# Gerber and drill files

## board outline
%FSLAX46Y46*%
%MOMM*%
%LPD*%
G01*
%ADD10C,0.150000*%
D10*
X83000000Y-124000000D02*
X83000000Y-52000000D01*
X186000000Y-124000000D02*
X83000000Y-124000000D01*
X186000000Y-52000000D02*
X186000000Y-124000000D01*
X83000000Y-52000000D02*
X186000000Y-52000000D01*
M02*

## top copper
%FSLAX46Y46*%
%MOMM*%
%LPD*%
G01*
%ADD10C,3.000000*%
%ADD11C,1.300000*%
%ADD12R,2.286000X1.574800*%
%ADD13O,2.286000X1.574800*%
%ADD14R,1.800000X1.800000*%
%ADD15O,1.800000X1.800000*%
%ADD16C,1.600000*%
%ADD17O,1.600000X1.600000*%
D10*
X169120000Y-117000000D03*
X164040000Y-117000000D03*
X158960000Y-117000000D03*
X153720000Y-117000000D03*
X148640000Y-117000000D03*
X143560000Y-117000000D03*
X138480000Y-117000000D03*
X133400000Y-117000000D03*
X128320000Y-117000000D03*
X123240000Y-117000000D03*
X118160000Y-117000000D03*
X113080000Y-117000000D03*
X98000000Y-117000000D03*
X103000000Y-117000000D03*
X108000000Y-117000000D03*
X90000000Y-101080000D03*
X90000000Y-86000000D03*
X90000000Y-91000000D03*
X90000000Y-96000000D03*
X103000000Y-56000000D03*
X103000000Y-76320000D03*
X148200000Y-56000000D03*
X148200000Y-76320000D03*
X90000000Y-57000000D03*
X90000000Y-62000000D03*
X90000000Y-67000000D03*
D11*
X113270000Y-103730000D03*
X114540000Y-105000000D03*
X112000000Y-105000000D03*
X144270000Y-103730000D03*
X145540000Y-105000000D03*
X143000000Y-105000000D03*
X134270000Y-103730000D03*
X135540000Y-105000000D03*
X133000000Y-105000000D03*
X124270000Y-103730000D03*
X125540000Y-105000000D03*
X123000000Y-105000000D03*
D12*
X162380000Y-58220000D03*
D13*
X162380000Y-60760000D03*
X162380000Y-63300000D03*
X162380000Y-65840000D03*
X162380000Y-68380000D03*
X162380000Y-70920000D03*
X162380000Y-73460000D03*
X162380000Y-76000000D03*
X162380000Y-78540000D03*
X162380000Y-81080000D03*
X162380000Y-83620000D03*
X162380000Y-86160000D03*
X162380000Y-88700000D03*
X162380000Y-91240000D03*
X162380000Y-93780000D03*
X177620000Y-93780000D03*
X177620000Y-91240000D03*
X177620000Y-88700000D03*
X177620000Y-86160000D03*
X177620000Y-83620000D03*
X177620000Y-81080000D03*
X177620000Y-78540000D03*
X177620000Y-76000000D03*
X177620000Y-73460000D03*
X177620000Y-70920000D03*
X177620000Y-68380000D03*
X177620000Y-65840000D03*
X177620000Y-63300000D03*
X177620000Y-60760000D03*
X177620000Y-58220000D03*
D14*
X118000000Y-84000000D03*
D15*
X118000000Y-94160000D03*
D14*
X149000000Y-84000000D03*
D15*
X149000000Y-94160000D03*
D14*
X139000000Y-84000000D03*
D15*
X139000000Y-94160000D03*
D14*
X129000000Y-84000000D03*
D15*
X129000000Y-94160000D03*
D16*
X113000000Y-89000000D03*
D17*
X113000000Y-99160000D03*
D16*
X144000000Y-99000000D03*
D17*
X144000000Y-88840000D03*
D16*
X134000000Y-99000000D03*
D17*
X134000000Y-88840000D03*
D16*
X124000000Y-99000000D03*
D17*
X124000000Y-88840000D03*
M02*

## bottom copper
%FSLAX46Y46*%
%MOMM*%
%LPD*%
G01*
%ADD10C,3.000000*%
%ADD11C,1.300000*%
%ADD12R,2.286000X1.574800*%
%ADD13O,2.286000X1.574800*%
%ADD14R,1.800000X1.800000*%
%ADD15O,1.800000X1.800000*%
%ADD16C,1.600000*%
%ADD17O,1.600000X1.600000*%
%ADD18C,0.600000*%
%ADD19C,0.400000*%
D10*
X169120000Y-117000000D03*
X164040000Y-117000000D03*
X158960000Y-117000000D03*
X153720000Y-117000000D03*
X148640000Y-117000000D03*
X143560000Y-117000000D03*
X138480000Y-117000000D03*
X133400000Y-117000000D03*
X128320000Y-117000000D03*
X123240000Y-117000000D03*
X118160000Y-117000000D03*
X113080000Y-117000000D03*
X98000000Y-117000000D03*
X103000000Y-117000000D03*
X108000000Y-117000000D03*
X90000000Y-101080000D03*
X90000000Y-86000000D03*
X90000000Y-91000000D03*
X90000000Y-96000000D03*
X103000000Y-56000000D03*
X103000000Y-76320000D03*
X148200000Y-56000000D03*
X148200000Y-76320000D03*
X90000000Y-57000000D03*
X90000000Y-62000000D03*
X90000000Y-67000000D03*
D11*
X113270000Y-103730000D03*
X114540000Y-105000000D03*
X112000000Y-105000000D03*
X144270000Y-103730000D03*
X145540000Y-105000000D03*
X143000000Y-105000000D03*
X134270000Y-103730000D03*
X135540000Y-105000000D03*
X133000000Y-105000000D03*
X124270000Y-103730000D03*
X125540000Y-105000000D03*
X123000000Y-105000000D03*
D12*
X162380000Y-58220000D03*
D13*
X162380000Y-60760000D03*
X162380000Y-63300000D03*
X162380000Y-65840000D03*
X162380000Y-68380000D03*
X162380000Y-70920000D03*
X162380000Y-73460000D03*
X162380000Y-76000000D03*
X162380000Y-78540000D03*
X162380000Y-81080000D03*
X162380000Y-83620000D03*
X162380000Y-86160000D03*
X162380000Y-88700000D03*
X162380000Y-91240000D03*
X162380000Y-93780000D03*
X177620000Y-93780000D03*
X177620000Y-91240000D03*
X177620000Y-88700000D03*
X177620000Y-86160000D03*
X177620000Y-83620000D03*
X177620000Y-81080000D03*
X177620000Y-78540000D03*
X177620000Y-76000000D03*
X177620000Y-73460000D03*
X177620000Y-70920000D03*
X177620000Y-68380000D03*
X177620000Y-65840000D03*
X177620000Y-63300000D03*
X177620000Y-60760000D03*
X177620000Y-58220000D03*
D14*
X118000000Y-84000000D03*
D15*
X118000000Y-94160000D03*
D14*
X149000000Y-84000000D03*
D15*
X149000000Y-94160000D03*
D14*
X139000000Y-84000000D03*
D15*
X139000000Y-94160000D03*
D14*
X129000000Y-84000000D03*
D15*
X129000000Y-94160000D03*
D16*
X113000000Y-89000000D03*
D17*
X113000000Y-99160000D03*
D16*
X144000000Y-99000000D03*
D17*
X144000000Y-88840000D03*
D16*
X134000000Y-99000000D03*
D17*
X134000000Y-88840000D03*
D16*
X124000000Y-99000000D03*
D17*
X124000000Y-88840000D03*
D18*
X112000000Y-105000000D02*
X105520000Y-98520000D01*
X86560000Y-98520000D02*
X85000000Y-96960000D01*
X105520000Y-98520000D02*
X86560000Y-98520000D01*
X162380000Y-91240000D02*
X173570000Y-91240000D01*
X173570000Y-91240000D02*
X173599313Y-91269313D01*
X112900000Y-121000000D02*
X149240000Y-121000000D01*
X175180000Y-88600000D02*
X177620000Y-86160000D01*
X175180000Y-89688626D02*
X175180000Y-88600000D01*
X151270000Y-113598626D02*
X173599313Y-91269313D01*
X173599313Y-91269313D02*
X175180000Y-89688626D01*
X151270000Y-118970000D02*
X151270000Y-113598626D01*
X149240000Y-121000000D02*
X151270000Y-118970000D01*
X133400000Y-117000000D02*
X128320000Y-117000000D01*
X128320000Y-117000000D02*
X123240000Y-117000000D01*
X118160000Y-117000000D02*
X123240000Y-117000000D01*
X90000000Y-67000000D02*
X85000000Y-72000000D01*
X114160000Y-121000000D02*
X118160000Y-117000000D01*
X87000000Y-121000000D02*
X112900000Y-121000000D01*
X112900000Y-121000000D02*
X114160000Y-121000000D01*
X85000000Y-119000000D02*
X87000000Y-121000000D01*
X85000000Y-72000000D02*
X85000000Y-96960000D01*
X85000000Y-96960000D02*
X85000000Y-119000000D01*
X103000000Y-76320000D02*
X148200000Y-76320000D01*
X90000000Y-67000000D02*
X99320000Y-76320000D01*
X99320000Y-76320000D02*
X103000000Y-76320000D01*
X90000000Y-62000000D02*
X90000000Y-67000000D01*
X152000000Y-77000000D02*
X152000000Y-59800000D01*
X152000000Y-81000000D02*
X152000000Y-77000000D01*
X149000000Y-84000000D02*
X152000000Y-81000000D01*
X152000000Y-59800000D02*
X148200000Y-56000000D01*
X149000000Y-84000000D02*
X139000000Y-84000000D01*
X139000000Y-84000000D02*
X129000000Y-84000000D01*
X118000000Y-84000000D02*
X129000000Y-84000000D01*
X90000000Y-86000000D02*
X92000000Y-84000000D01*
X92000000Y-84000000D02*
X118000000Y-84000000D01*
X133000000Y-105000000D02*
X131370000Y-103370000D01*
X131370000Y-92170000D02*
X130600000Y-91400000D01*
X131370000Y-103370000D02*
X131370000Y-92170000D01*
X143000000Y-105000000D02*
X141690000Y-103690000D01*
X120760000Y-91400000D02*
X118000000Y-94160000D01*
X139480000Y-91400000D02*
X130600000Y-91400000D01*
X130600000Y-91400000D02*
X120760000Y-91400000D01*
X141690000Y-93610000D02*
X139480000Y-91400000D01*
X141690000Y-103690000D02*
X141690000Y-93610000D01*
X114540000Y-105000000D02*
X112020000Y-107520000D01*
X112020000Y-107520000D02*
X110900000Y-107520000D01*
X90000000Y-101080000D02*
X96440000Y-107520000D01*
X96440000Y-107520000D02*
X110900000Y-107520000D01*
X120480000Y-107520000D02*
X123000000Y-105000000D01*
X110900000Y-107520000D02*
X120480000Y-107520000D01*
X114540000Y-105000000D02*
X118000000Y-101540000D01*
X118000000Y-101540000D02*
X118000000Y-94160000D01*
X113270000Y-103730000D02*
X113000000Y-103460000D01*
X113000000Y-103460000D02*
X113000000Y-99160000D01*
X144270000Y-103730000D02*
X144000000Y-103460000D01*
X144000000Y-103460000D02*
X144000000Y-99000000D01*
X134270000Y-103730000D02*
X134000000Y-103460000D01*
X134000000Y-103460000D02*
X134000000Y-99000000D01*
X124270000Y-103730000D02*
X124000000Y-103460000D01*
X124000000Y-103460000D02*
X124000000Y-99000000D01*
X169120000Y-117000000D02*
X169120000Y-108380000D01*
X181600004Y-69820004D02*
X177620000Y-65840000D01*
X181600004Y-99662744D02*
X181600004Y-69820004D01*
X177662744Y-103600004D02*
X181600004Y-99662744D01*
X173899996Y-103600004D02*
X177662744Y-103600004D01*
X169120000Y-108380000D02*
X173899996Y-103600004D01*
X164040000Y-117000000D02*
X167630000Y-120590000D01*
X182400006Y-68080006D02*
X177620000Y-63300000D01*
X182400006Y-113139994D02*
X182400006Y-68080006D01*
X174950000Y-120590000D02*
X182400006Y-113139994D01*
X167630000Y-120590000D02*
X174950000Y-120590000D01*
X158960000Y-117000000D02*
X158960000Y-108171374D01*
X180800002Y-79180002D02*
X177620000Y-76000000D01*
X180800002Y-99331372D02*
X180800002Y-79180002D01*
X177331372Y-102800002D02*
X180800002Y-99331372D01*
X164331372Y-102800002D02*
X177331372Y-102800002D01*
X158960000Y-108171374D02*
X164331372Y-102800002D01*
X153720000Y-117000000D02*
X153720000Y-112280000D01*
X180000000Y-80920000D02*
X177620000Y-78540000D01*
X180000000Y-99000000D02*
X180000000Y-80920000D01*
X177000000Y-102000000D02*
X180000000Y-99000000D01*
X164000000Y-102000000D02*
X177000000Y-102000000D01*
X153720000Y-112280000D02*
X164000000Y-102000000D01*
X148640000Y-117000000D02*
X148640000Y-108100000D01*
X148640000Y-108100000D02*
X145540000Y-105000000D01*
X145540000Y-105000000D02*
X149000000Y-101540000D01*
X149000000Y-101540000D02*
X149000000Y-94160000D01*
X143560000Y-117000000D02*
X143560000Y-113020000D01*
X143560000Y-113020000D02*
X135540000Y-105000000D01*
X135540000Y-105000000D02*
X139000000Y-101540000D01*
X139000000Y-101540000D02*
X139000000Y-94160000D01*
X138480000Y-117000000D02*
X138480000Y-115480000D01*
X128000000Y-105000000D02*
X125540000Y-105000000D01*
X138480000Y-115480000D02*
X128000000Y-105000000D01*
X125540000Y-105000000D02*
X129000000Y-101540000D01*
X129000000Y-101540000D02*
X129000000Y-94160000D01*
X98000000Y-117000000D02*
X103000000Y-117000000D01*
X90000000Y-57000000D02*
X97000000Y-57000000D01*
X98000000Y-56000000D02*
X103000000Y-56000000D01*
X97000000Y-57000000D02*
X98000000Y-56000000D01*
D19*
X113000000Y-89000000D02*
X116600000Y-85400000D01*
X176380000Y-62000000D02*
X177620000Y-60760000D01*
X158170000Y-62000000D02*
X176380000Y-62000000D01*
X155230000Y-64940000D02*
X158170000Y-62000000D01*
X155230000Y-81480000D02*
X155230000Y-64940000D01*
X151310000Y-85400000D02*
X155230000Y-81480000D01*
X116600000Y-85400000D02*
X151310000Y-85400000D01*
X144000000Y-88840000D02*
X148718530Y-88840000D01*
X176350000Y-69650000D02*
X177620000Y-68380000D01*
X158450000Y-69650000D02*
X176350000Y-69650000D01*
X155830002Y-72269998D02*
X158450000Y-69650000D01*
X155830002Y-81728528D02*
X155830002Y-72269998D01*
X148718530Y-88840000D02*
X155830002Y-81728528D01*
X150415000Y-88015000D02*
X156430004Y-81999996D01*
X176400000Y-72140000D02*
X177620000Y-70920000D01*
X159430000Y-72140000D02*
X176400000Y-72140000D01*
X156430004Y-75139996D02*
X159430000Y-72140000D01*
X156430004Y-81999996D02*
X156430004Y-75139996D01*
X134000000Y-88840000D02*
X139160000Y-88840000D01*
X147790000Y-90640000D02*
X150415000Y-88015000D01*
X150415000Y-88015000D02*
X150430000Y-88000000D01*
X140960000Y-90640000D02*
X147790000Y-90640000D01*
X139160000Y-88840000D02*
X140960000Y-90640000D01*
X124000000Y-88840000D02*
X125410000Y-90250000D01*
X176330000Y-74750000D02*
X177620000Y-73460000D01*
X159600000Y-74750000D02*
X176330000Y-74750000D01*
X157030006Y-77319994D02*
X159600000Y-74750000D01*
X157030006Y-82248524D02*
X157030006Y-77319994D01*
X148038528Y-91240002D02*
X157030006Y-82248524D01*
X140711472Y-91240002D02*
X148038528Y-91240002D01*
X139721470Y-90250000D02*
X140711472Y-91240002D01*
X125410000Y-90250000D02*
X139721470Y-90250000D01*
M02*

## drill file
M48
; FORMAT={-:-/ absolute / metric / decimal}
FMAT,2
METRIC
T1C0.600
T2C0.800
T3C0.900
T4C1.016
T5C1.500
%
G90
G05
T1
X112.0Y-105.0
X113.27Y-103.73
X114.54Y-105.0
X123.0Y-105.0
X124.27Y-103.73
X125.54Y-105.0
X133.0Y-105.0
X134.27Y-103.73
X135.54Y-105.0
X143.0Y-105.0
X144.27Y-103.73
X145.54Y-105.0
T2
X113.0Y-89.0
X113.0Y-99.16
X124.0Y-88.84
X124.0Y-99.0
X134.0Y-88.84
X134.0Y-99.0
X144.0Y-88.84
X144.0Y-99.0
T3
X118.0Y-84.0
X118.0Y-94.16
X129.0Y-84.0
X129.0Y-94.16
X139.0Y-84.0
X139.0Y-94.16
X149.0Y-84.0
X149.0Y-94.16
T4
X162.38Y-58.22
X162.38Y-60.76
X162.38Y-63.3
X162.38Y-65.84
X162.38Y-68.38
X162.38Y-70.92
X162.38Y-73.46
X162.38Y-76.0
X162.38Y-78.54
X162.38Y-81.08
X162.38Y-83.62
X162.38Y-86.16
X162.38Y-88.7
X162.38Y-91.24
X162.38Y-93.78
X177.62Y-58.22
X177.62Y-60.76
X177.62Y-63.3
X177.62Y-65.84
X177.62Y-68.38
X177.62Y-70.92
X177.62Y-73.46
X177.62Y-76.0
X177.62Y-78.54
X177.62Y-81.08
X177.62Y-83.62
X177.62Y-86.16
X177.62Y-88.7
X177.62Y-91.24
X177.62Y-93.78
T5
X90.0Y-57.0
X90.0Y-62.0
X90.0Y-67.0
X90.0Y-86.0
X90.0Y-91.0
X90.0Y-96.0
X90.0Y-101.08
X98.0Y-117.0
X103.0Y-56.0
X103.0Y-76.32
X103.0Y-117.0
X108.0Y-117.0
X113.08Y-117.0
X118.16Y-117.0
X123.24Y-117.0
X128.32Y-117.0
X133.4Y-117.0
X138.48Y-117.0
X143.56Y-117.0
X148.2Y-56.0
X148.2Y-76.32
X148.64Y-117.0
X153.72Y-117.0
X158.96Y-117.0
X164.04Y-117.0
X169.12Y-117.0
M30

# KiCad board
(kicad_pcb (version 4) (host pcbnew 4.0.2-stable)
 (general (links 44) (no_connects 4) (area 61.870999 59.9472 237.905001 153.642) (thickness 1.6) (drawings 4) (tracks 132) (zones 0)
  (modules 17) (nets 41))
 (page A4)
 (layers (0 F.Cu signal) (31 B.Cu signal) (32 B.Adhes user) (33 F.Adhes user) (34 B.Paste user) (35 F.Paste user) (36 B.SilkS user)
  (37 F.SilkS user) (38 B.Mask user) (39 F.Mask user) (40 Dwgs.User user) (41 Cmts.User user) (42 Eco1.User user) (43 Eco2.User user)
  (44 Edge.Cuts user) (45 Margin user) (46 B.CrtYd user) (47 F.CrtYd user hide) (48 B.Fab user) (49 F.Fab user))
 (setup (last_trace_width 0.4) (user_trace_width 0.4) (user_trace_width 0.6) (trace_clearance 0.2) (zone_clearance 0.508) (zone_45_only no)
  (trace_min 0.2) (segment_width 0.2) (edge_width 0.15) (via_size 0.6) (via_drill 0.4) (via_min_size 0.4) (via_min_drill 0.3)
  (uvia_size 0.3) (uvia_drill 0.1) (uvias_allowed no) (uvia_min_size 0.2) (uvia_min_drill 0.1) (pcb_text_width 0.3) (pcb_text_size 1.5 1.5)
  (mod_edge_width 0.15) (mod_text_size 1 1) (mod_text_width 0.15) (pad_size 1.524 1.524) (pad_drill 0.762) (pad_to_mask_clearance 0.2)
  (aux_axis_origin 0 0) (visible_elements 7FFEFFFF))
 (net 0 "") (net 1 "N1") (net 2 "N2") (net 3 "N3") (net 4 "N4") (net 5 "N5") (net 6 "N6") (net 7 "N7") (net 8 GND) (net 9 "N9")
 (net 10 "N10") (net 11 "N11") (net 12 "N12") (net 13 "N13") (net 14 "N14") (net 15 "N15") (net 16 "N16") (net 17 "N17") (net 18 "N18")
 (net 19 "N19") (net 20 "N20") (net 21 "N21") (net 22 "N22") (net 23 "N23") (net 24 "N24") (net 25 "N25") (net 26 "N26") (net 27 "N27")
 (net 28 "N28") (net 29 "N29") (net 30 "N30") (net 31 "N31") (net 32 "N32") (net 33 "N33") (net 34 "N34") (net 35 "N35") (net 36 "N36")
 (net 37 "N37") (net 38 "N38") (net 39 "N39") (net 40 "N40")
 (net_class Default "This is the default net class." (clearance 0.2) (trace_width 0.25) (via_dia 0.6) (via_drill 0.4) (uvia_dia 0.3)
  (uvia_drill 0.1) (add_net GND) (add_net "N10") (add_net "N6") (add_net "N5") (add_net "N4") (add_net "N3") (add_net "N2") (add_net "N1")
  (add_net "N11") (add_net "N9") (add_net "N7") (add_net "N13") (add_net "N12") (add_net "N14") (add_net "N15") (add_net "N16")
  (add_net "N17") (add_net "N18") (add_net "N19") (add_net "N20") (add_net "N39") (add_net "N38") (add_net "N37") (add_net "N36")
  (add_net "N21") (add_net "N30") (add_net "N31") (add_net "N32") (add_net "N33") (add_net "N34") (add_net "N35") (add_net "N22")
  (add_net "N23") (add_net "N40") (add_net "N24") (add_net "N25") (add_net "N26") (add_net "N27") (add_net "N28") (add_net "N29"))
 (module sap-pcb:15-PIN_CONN (layer F.Cu) (at 98 117)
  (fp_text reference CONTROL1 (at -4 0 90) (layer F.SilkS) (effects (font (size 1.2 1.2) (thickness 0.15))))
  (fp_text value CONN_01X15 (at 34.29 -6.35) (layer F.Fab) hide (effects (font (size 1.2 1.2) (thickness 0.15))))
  (pad 15 thru_hole circle (at 71.12 0) (size 3 3) (drill 1.5) (layers *.Cu *.Mask F.SilkS) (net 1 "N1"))
  (pad 14 thru_hole circle (at 66.04 0) (size 3 3) (drill 1.5) (layers *.Cu *.Mask F.SilkS) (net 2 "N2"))
  (pad 13 thru_hole circle (at 60.96 0) (size 3 3) (drill 1.5) (layers *.Cu *.Mask F.SilkS) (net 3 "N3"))
  (pad 12 thru_hole circle (at 55.72 0) (size 3 3) (drill 1.5) (layers *.Cu *.Mask F.SilkS) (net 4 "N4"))
  (pad 11 thru_hole circle (at 50.64 0) (size 3 3) (drill 1.5) (layers *.Cu *.Mask F.SilkS) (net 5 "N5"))
  (pad 10 thru_hole circle (at 45.56 0) (size 3 3) (drill 1.5) (layers *.Cu *.Mask F.SilkS) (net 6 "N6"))
  (pad 9 thru_hole circle (at 40.48 0) (size 3 3) (drill 1.5) (layers *.Cu *.Mask F.SilkS) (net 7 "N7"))
  (pad 8 thru_hole circle (at 35.4 0) (size 3 3) (drill 1.5) (layers *.Cu *.Mask F.SilkS) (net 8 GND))
  (pad 7 thru_hole circle (at 30.32 0) (size 3 3) (drill 1.5) (layers *.Cu *.Mask F.SilkS) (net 8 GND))
  (pad 6 thru_hole circle (at 25.24 0) (size 3 3) (drill 1.5) (layers *.Cu *.Mask F.SilkS) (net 8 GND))
  (pad 5 thru_hole circle (at 20.16 0) (size 3 3) (drill 1.5) (layers *.Cu *.Mask F.SilkS) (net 8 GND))
  (pad 4 thru_hole circle (at 15.08 0) (size 3 3) (drill 1.5) (layers *.Cu *.Mask F.SilkS) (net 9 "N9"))
  (pad 1 thru_hole circle (at 0 0) (size 3 3) (drill 1.5) (layers *.Cu *.Mask F.SilkS) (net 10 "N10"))
  (pad 2 thru_hole circle (at 5 0) (size 3 3) (drill 1.5) (layers *.Cu *.Mask F.SilkS) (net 10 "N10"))
  (pad 3 thru_hole circle (at 10 0) (size 3 3) (drill 1.5) (layers *.Cu *.Mask F.SilkS) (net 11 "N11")))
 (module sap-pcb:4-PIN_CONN (layer F.Cu) (at 90 86 270)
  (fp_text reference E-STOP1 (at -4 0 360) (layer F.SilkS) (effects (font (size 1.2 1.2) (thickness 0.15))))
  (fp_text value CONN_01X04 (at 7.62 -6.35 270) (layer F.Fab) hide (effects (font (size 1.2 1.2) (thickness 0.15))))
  (pad 4 thru_hole circle (at 15.08 0 270) (size 3 3) (drill 1.5) (layers *.Cu *.Mask F.SilkS) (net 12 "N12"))
  (pad 1 thru_hole circle (at 0 0 270) (size 3 3) (drill 1.5) (layers *.Cu *.Mask F.SilkS) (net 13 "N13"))
  (pad 2 thru_hole circle (at 5 0 270) (size 3 3) (drill 1.5) (layers *.Cu *.Mask F.SilkS) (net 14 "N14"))
  (pad 3 thru_hole circle (at 10 0 270) (size 3 3) (drill 1.5) (layers *.Cu *.Mask F.SilkS) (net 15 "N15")))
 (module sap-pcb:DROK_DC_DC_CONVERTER (layer F.Cu) (at 103 56)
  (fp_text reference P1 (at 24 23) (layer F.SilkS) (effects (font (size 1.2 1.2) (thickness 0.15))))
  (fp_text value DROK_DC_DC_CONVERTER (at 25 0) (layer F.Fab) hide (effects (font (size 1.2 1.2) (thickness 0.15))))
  (pad 1 thru_hole circle (at 0 0) (size 3 3) (drill 1.5) (layers *.Cu *.Mask F.SilkS) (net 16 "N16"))
  (pad 2 thru_hole circle (at 0 20.32) (size 3 3) (drill 1.5) (layers *.Cu *.Mask F.SilkS) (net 8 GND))
  (pad 3 thru_hole circle (at 45.2 0) (size 3 3) (drill 1.5) (layers *.Cu *.Mask F.SilkS) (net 13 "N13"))
  (pad 4 thru_hole circle (at 45.2 20.32) (size 3 3) (drill 1.5) (layers *.Cu *.Mask F.SilkS) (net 8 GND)))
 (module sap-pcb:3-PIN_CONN (layer F.Cu) (at 90 57 270)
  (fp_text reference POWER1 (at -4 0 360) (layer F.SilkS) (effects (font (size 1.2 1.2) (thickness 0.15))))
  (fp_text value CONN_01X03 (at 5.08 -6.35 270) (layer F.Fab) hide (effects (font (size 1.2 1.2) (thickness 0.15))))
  (pad 1 thru_hole circle (at 0 0 270) (size 3 3) (drill 1.5) (layers *.Cu *.Mask F.SilkS) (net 16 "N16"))
  (pad 2 thru_hole circle (at 5 0 270) (size 3 3) (drill 1.5) (layers *.Cu *.Mask F.SilkS) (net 8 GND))
  (pad 3 thru_hole circle (at 10 0 270) (size 3 3) (drill 1.5) (layers *.Cu *.Mask F.SilkS) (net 8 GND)))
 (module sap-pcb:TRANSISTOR (layer F.Cu) (at 112 105)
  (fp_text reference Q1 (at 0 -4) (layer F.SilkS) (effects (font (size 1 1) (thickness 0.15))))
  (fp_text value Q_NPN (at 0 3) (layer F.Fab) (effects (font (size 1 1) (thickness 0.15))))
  (pad 2 thru_hole circle (at 1.27 -1.27 90) (size 1.3 1.3) (drill 0.6) (layers *.Cu *.Mask F.SilkS) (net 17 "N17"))
  (pad 3 thru_hole circle (at 2.54 0 90) (size 1.3 1.3) (drill 0.6) (layers *.Cu *.Mask F.SilkS) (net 12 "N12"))
  (pad 1 thru_hole circle (at 0 0 90) (size 1.3 1.3) (drill 0.6) (layers *.Cu *.Mask F.SilkS) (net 8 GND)))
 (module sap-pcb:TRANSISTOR (layer F.Cu) (at 143 105)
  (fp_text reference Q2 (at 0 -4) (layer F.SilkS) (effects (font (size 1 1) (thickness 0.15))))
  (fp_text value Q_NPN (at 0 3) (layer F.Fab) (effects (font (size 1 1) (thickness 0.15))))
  (pad 2 thru_hole circle (at 1.27 -1.27 90) (size 1.3 1.3) (drill 0.6) (layers *.Cu *.Mask F.SilkS) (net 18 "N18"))
  (pad 3 thru_hole circle (at 2.54 0 90) (size 1.3 1.3) (drill 0.6) (layers *.Cu *.Mask F.SilkS) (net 5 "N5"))
  (pad 1 thru_hole circle (at 0 0 90) (size 1.3 1.3) (drill 0.6) (layers *.Cu *.Mask F.SilkS) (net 12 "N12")))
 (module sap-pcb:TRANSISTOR (layer F.Cu) (at 133 105)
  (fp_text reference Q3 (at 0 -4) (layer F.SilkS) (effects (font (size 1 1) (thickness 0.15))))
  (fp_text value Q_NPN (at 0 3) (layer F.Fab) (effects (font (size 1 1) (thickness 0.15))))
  (pad 2 thru_hole circle (at 1.27 -1.27 90) (size 1.3 1.3) (drill 0.6) (layers *.Cu *.Mask F.SilkS) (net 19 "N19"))
  (pad 3 thru_hole circle (at 2.54 0 90) (size 1.3 1.3) (drill 0.6) (layers *.Cu *.Mask F.SilkS) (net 6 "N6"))
  (pad 1 thru_hole circle (at 0 0 90) (size 1.3 1.3) (drill 0.6) (layers *.Cu *.Mask F.SilkS) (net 12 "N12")))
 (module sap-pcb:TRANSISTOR (layer F.Cu) (at 123 105)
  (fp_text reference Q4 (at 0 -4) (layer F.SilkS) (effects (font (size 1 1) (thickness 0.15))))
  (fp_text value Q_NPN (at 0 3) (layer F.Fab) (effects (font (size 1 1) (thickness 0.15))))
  (pad 2 thru_hole circle (at 1.27 -1.27 90) (size 1.3 1.3) (drill 0.6) (layers *.Cu *.Mask F.SilkS) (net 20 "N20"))
  (pad 3 thru_hole circle (at 2.54 0 90) (size 1.3 1.3) (drill 0.6) (layers *.Cu *.Mask F.SilkS) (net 7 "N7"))
  (pad 1 thru_hole circle (at 0 0 90) (size 1.3 1.3) (drill 0.6) (layers *.Cu *.Mask F.SilkS) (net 12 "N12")))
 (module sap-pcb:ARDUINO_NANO (layer F.Cu) (at 170 76 270)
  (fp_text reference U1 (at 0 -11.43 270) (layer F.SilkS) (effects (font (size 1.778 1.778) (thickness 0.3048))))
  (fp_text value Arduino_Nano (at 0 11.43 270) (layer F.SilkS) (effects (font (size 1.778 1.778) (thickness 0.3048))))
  (pad 1 thru_hole rect (at -17.78 7.62 270) (size 1.5748 2.286) (drill 1.016) (layers *.Cu *.Mask F.SilkS) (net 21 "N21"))
  (pad 2 thru_hole oval (at -15.24 7.62 270) (size 1.5748 2.286) (drill 1.016) (layers *.Cu *.Mask F.SilkS) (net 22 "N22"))
  (pad 3 thru_hole oval (at -12.7 7.62 270) (size 1.5748 2.286) (drill 1.016) (layers *.Cu *.Mask F.SilkS) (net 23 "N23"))
  (pad 4 thru_hole oval (at -10.16 7.62 270) (size 1.5748 2.286) (drill 1.016) (layers *.Cu *.Mask F.SilkS) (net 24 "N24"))
  (pad 5 thru_hole oval (at -7.62 7.62 270) (size 1.5748 2.286) (drill 1.016) (layers *.Cu *.Mask F.SilkS) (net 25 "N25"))
  (pad 6 thru_hole oval (at -5.08 7.62 270) (size 1.5748 2.286) (drill 1.016) (layers *.Cu *.Mask F.SilkS) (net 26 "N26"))
  (pad 7 thru_hole oval (at -2.54 7.62 270) (size 1.5748 2.286) (drill 1.016) (layers *.Cu *.Mask F.SilkS) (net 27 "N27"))
  (pad 8 thru_hole oval (at 0 7.62 270) (size 1.5748 2.286) (drill 1.016) (layers *.Cu *.Mask F.SilkS) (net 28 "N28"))
  (pad 9 thru_hole oval (at 2.54 7.62 270) (size 1.5748 2.286) (drill 1.016) (layers *.Cu *.Mask F.SilkS) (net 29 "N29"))
  (pad 10 thru_hole oval (at 5.08 7.62 270) (size 1.5748 2.286) (drill 1.016) (layers *.Cu *.Mask F.SilkS) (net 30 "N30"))
  (pad 11 thru_hole oval (at 7.62 7.62 270) (size 1.5748 2.286) (drill 1.016) (layers *.Cu *.Mask F.SilkS) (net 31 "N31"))
  (pad 12 thru_hole oval (at 10.16 7.62 270) (size 1.5748 2.286) (drill 1.016) (layers *.Cu *.Mask F.SilkS) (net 10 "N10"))
  (pad 13 thru_hole oval (at 12.7 7.62 270) (size 1.5748 2.286) (drill 1.016) (layers *.Cu *.Mask F.SilkS) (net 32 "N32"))
  (pad 14 thru_hole oval (at 15.24 7.62 270) (size 1.5748 2.286) (drill 1.016) (layers *.Cu *.Mask F.SilkS) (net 8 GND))
  (pad 15 thru_hole oval (at 17.78 7.62 270) (size 1.5748 2.286) (drill 1.016) (layers *.Cu *.Mask F.SilkS) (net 16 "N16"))
  (pad 16 thru_hole oval (at 17.78 -7.62 270) (size 1.5748 2.286) (drill 1.016) (layers *.Cu *.Mask F.SilkS) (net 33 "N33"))
  (pad 17 thru_hole oval (at 15.24 -7.62 270) (size 1.5748 2.286) (drill 1.016) (layers *.Cu *.Mask F.SilkS) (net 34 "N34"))
  (pad 18 thru_hole oval (at 12.7 -7.62 270) (size 1.5748 2.286) (drill 1.016) (layers *.Cu *.Mask F.SilkS) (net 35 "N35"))
  (pad 19 thru_hole oval (at 10.16 -7.62 270) (size 1.5748 2.286) (drill 1.016) (layers *.Cu *.Mask F.SilkS) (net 8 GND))
  (pad 20 thru_hole oval (at 7.62 -7.62 270) (size 1.5748 2.286) (drill 1.016) (layers *.Cu *.Mask F.SilkS) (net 11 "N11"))
  (pad 21 thru_hole oval (at 5.08 -7.62 270) (size 1.5748 2.286) (drill 1.016) (layers *.Cu *.Mask F.SilkS) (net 9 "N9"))
  (pad 22 thru_hole oval (at 2.54 -7.62 270) (size 1.5748 2.286) (drill 1.016) (layers *.Cu *.Mask F.SilkS) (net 4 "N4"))
  (pad 23 thru_hole oval (at 0 -7.62 270) (size 1.5748 2.286) (drill 1.016) (layers *.Cu *.Mask F.SilkS) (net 3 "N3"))
  (pad 24 thru_hole oval (at -2.54 -7.62 270) (size 1.5748 2.286) (drill 1.016) (layers *.Cu *.Mask F.SilkS) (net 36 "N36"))
  (pad 25 thru_hole oval (at -5.08 -7.62 270) (size 1.5748 2.286) (drill 1.016) (layers *.Cu *.Mask F.SilkS) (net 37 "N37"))
  (pad 26 thru_hole oval (at -7.62 -7.62 270) (size 1.5748 2.286) (drill 1.016) (layers *.Cu *.Mask F.SilkS) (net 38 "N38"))
  (pad 27 thru_hole oval (at -10.16 -7.62 270) (size 1.5748 2.286) (drill 1.016) (layers *.Cu *.Mask F.SilkS) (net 1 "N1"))
  (pad 28 thru_hole oval (at -12.7 -7.62 270) (size 1.5748 2.286) (drill 1.016) (layers *.Cu *.Mask F.SilkS) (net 2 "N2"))
  (pad 29 thru_hole oval (at -15.24 -7.62 270) (size 1.5748 2.286) (drill 1.016) (layers *.Cu *.Mask F.SilkS) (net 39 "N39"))
  (pad 30 thru_hole oval (at -17.78 -7.62 270) (size 1.5748 2.286) (drill 1.016) (layers *.Cu *.Mask F.SilkS) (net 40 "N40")))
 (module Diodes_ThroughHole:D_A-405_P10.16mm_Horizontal (layer F.Cu) (at 118 84 270)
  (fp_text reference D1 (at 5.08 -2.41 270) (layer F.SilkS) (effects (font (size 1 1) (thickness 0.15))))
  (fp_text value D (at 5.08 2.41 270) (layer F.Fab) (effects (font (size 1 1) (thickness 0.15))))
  (pad 1 thru_hole rect (at 0 0 270) (size 1.8 1.8) (drill 0.9) (layers *.Cu *.Mask) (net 13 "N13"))
  (pad 2 thru_hole oval (at 10.16 0 270) (size 1.8 1.8) (drill 0.9) (layers *.Cu *.Mask) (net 12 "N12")))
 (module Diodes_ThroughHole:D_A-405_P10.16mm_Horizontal (layer F.Cu) (at 149 84 270)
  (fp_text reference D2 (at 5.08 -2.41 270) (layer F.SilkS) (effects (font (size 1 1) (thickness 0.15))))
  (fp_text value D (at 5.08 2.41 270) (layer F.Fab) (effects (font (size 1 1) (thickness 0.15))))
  (pad 1 thru_hole rect (at 0 0 270) (size 1.8 1.8) (drill 0.9) (layers *.Cu *.Mask) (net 13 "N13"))
  (pad 2 thru_hole oval (at 10.16 0 270) (size 1.8 1.8) (drill 0.9) (layers *.Cu *.Mask) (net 5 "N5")))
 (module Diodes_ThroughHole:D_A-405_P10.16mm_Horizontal (layer F.Cu) (at 139 84 270)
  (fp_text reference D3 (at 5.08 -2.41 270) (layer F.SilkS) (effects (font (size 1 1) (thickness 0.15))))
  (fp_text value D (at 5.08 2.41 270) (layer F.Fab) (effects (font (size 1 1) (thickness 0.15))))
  (pad 1 thru_hole rect (at 0 0 270) (size 1.8 1.8) (drill 0.9) (layers *.Cu *.Mask) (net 13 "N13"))
  (pad 2 thru_hole oval (at 10.16 0 270) (size 1.8 1.8) (drill 0.9) (layers *.Cu *.Mask) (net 6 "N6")))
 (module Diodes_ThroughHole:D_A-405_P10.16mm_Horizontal (layer F.Cu) (at 129 84 270)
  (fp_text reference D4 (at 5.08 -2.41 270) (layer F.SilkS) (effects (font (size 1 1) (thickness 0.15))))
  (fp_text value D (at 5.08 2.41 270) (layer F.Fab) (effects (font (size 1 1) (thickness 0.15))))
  (pad 1 thru_hole rect (at 0 0 270) (size 1.8 1.8) (drill 0.9) (layers *.Cu *.Mask) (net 13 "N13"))
  (pad 2 thru_hole oval (at 10.16 0 270) (size 1.8 1.8) (drill 0.9) (layers *.Cu *.Mask) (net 7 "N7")))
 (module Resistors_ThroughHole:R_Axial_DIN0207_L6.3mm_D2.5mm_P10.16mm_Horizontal (layer F.Cu) (at 113 89 270)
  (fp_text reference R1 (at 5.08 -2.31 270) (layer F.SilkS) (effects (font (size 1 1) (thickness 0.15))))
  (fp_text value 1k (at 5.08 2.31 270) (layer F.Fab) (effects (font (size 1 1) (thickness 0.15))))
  (pad 1 thru_hole circle (at 0 0 270) (size 1.6 1.6) (drill 0.8) (layers *.Cu *.Mask) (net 39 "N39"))
  (pad 2 thru_hole oval (at 10.16 0 270) (size 1.6 1.6) (drill 0.8) (layers *.Cu *.Mask) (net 17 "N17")))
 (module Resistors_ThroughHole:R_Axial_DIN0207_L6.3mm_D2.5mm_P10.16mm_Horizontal (layer F.Cu) (at 144 99 90)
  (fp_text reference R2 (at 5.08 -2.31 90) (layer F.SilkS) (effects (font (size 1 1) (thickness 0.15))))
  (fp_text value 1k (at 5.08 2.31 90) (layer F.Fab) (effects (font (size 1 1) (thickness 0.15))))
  (pad 1 thru_hole circle (at 0 0 90) (size 1.6 1.6) (drill 0.8) (layers *.Cu *.Mask) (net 18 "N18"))
  (pad 2 thru_hole oval (at 10.16 0 90) (size 1.6 1.6) (drill 0.8) (layers *.Cu *.Mask) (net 38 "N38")))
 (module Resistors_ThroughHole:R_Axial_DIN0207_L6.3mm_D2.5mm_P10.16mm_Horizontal (layer F.Cu) (at 134 99 90)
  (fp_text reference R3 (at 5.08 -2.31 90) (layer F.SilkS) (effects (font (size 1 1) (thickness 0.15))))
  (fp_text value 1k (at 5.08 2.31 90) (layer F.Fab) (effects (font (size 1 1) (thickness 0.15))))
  (pad 1 thru_hole circle (at 0 0 90) (size 1.6 1.6) (drill 0.8) (layers *.Cu *.Mask) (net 19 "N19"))
  (pad 2 thru_hole oval (at 10.16 0 90) (size 1.6 1.6) (drill 0.8) (layers *.Cu *.Mask) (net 37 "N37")))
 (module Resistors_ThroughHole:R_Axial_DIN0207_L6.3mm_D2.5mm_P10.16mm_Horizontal (layer F.Cu) (at 124 99 90)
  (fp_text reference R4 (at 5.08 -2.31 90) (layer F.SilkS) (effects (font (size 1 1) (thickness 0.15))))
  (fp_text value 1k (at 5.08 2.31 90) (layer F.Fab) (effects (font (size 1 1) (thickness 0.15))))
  (pad 1 thru_hole circle (at 0 0 90) (size 1.6 1.6) (drill 0.8) (layers *.Cu *.Mask) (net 20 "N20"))
  (pad 2 thru_hole oval (at 10.16 0 90) (size 1.6 1.6) (drill 0.8) (layers *.Cu *.Mask) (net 36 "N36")))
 (gr_line (start 83 124) (end 83 52) (angle 90) (layer Edge.Cuts) (width 0.15))
 (gr_line (start 186 124) (end 83 124) (angle 90) (layer Edge.Cuts) (width 0.15))
 (gr_line (start 186 52) (end 186 124) (angle 90) (layer Edge.Cuts) (width 0.15))
 (gr_line (start 83 52) (end 186 52) (angle 90) (layer Edge.Cuts) (width 0.15))
 (segment (start 112 105) (end 105.52 98.52) (width 0.6) (layer B.Cu) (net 8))
 (segment (start 86.56 98.52) (end 85 96.96) (width 0.6) (layer B.Cu) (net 8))
 (segment (start 105.52 98.52) (end 86.56 98.52) (width 0.6) (layer B.Cu) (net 8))
 (segment (start 162.38 91.24) (end 173.57 91.24) (width 0.6) (layer B.Cu) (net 8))
 (segment (start 173.57 91.24) (end 173.599313 91.269313) (width 0.6) (layer B.Cu) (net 8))
 (segment (start 112.9 121) (end 149.24 121) (width 0.6) (layer B.Cu) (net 8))
 (segment (start 175.18 88.6) (end 177.62 86.16) (width 0.6) (layer B.Cu) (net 8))
 (segment (start 175.18 89.688626) (end 175.18 88.6) (width 0.6) (layer B.Cu) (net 8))
 (segment (start 151.27 113.598626) (end 173.599313 91.269313) (width 0.6) (layer B.Cu) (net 8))
 (segment (start 173.599313 91.269313) (end 175.18 89.688626) (width 0.6) (layer B.Cu) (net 8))
 (segment (start 151.27 118.97) (end 151.27 113.598626) (width 0.6) (layer B.Cu) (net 8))
 (segment (start 149.24 121) (end 151.27 118.97) (width 0.6) (layer B.Cu) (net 8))
 (segment (start 133.4 117) (end 128.32 117) (width 0.6) (layer B.Cu) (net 8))
 (segment (start 128.32 117) (end 123.24 117) (width 0.6) (layer B.Cu) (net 8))
 (segment (start 118.16 117) (end 123.24 117) (width 0.6) (layer B.Cu) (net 8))
 (segment (start 90 67) (end 85 72) (width 0.6) (layer B.Cu) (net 8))
 (segment (start 114.16 121) (end 118.16 117) (width 0.6) (layer B.Cu) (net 8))
 (segment (start 87 121) (end 112.9 121) (width 0.6) (layer B.Cu) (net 8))
 (segment (start 112.9 121) (end 114.16 121) (width 0.6) (layer B.Cu) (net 8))
 (segment (start 85 119) (end 87 121) (width 0.6) (layer B.Cu) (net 8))
 (segment (start 85 72) (end 85 96.96) (width 0.6) (layer B.Cu) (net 8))
 (segment (start 85 96.96) (end 85 119) (width 0.6) (layer B.Cu) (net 8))
 (segment (start 103 76.32) (end 148.2 76.32) (width 0.6) (layer B.Cu) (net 8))
 (segment (start 90 67) (end 99.32 76.32) (width 0.6) (layer B.Cu) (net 8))
 (segment (start 99.32 76.32) (end 103 76.32) (width 0.6) (layer B.Cu) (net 8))
 (segment (start 90 62) (end 90 67) (width 0.6) (layer B.Cu) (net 8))
 (segment (start 152 77) (end 152 59.8) (width 0.6) (layer B.Cu) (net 13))
 (segment (start 152 81) (end 152 77) (width 0.6) (layer B.Cu) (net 13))
 (segment (start 149 84) (end 152 81) (width 0.6) (layer B.Cu) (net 13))
 (segment (start 152 59.8) (end 148.2 56) (width 0.6) (layer B.Cu) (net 13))
 (segment (start 149 84) (end 139 84) (width 0.6) (layer B.Cu) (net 13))
 (segment (start 139 84) (end 129 84) (width 0.6) (layer B.Cu) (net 13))
 (segment (start 118 84) (end 129 84) (width 0.6) (layer B.Cu) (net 13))
 (segment (start 90 86) (end 92 84) (width 0.6) (layer B.Cu) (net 13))
 (segment (start 92 84) (end 118 84) (width 0.6) (layer B.Cu) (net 13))
 (segment (start 133 105) (end 131.37 103.37) (width 0.6) (layer B.Cu) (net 12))
 (segment (start 131.37 92.17) (end 130.6 91.4) (width 0.6) (layer B.Cu) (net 12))
 (segment (start 131.37 103.37) (end 131.37 92.17) (width 0.6) (layer B.Cu) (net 12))
 (segment (start 143 105) (end 141.69 103.69) (width 0.6) (layer B.Cu) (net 12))
 (segment (start 120.76 91.4) (end 118 94.16) (width 0.6) (layer B.Cu) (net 12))
 (segment (start 139.48 91.4) (end 130.6 91.4) (width 0.6) (layer B.Cu) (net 12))
 (segment (start 130.6 91.4) (end 120.76 91.4) (width 0.6) (layer B.Cu) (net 12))
 (segment (start 141.69 93.61) (end 139.48 91.4) (width 0.6) (layer B.Cu) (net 12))
 (segment (start 141.69 103.69) (end 141.69 93.61) (width 0.6) (layer B.Cu) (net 12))
 (segment (start 114.54 105) (end 112.02 107.52) (width 0.6) (layer B.Cu) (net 12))
 (segment (start 112.02 107.52) (end 110.9 107.52) (width 0.6) (layer B.Cu) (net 12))
 (segment (start 90 101.08) (end 96.44 107.52) (width 0.6) (layer B.Cu) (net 12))
 (segment (start 96.44 107.52) (end 110.9 107.52) (width 0.6) (layer B.Cu) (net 12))
 (segment (start 120.48 107.52) (end 123 105) (width 0.6) (layer B.Cu) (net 12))
 (segment (start 110.9 107.52) (end 120.48 107.52) (width 0.6) (layer B.Cu) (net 12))
 (segment (start 114.54 105) (end 118 101.54) (width 0.6) (layer B.Cu) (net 12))
 (segment (start 118 101.54) (end 118 94.16) (width 0.6) (layer B.Cu) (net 12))
 (segment (start 113.27 103.73) (end 113 103.46) (width 0.6) (layer B.Cu) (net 17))
 (segment (start 113 103.46) (end 113 99.16) (width 0.6) (layer B.Cu) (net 17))
 (segment (start 144.27 103.73) (end 144 103.46) (width 0.6) (layer B.Cu) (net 18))
 (segment (start 144 103.46) (end 144 99) (width 0.6) (layer B.Cu) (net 18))
 (segment (start 134.27 103.73) (end 134 103.46) (width 0.6) (layer B.Cu) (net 19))
 (segment (start 134 103.46) (end 134 99) (width 0.6) (layer B.Cu) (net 19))
 (segment (start 124.27 103.73) (end 124 103.46) (width 0.6) (layer B.Cu) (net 20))
 (segment (start 124 103.46) (end 124 99) (width 0.6) (layer B.Cu) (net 20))
 (segment (start 169.12 117) (end 169.12 108.38) (width 0.6) (layer B.Cu) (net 1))
 (segment (start 181.600004 69.820004) (end 177.62 65.84) (width 0.6) (layer B.Cu) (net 1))
 (segment (start 181.600004 99.662744) (end 181.600004 69.820004) (width 0.6) (layer B.Cu) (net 1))
 (segment (start 177.662744 103.600004) (end 181.600004 99.662744) (width 0.6) (layer B.Cu) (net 1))
 (segment (start 173.899996 103.600004) (end 177.662744 103.600004) (width 0.6) (layer B.Cu) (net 1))
 (segment (start 169.12 108.38) (end 173.899996 103.600004) (width 0.6) (layer B.Cu) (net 1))
 (segment (start 164.04 117) (end 167.63 120.59) (width 0.6) (layer B.Cu) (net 2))
 (segment (start 182.400006 68.080006) (end 177.62 63.3) (width 0.6) (layer B.Cu) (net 2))
 (segment (start 182.400006 113.139994) (end 182.400006 68.080006) (width 0.6) (layer B.Cu) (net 2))
 (segment (start 174.95 120.59) (end 182.400006 113.139994) (width 0.6) (layer B.Cu) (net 2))
 (segment (start 167.63 120.59) (end 174.95 120.59) (width 0.6) (layer B.Cu) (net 2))
 (segment (start 158.96 117) (end 158.96 108.171374) (width 0.6) (layer B.Cu) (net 3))
 (segment (start 180.800002 79.180002) (end 177.62 76) (width 0.6) (layer B.Cu) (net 3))
 (segment (start 180.800002 99.331372) (end 180.800002 79.180002) (width 0.6) (layer B.Cu) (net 3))
 (segment (start 177.331372 102.800002) (end 180.800002 99.331372) (width 0.6) (layer B.Cu) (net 3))
 (segment (start 164.331372 102.800002) (end 177.331372 102.800002) (width 0.6) (layer B.Cu) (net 3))
 (segment (start 158.96 108.171374) (end 164.331372 102.800002) (width 0.6) (layer B.Cu) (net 3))
 (segment (start 153.72 117) (end 153.72 112.28) (width 0.6) (layer B.Cu) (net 4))
 (segment (start 180 80.92) (end 177.62 78.54) (width 0.6) (layer B.Cu) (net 4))
 (segment (start 180 99) (end 180 80.92) (width 0.6) (layer B.Cu) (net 4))
 (segment (start 177 102) (end 180 99) (width 0.6) (layer B.Cu) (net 4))
 (segment (start 164 102) (end 177 102) (width 0.6) (layer B.Cu) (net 4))
 (segment (start 153.72 112.28) (end 164 102) (width 0.6) (layer B.Cu) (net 4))
 (segment (start 148.64 117) (end 148.64 108.1) (width 0.6) (layer B.Cu) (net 5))
 (segment (start 148.64 108.1) (end 145.54 105) (width 0.6) (layer B.Cu) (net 5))
 (segment (start 145.54 105) (end 149 101.54) (width 0.6) (layer B.Cu) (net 5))
 (segment (start 149 101.54) (end 149 94.16) (width 0.6) (layer B.Cu) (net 5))
 (segment (start 143.56 117) (end 143.56 113.02) (width 0.6) (layer B.Cu) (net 6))
 (segment (start 143.56 113.02) (end 135.54 105) (width 0.6) (layer B.Cu) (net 6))
 (segment (start 135.54 105) (end 139 101.54) (width 0.6) (layer B.Cu) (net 6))
 (segment (start 139 101.54) (end 139 94.16) (width 0.6) (layer B.Cu) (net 6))
 (segment (start 138.48 117) (end 138.48 115.48) (width 0.6) (layer B.Cu) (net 7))
 (segment (start 128 105) (end 125.54 105) (width 0.6) (layer B.Cu) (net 7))
 (segment (start 138.48 115.48) (end 128 105) (width 0.6) (layer B.Cu) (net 7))
 (segment (start 125.54 105) (end 129 101.54) (width 0.6) (layer B.Cu) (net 7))
 (segment (start 129 101.54) (end 129 94.16) (width 0.6) (layer B.Cu) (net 7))
 (segment (start 98 117) (end 103 117) (width 0.6) (layer B.Cu) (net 10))
 (segment (start 90 57) (end 97 57) (width 0.6) (layer B.Cu) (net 16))
 (segment (start 98 56) (end 103 56) (width 0.6) (layer B.Cu) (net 16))
 (segment (start 97 57) (end 98 56) (width 0.6) (layer B.Cu) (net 16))
 (segment (start 113 89) (end 116.6 85.4) (width 0.4) (layer B.Cu) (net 39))
 (segment (start 176.38 62) (end 177.62 60.76) (width 0.4) (layer B.Cu) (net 39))
 (segment (start 158.17 62) (end 176.38 62) (width 0.4) (layer B.Cu) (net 39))
 (segment (start 155.23 64.94) (end 158.17 62) (width 0.4) (layer B.Cu) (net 39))
 (segment (start 155.23 81.48) (end 155.23 64.94) (width 0.4) (layer B.Cu) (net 39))
 (segment (start 151.31 85.4) (end 155.23 81.48) (width 0.4) (layer B.Cu) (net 39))
 (segment (start 116.6 85.4) (end 151.31 85.4) (width 0.4) (layer B.Cu) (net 39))
 (segment (start 144 88.84) (end 148.71853 88.84) (width 0.4) (layer B.Cu) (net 38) (status 400000))
 (segment (start 176.35 69.65) (end 177.62 68.38) (width 0.4) (layer B.Cu) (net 38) (status 800000))
 (segment (start 158.45 69.65) (end 176.35 69.65) (width 0.4) (layer B.Cu) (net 38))
 (segment (start 155.830002 72.269998) (end 158.45 69.65) (width 0.4) (layer B.Cu) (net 38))
 (segment (start 155.830002 81.728528) (end 155.830002 72.269998) (width 0.4) (layer B.Cu) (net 38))
 (segment (start 148.71853 88.84) (end 155.830002 81.728528) (width 0.4) (layer B.Cu) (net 38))
 (segment (start 150.415 88.015) (end 156.430004 81.999996) (width 0.4) (layer B.Cu) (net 37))
 (segment (start 176.4 72.14) (end 177.62 70.92) (width 0.4) (layer B.Cu) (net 37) (status 800000))
 (segment (start 159.43 72.14) (end 176.4 72.14) (width 0.4) (layer B.Cu) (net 37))
 (segment (start 156.430004 75.139996) (end 159.43 72.14) (width 0.4) (layer B.Cu) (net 37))
 (segment (start 156.430004 81.999996) (end 156.430004 75.139996) (width 0.4) (layer B.Cu) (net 37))
 (segment (start 134 88.84) (end 139.16 88.84) (width 0.4) (layer B.Cu) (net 37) (status 400000))
 (segment (start 147.79 90.64) (end 150.415 88.015) (width 0.4) (layer B.Cu) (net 37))
 (segment (start 150.415 88.015) (end 150.43 88) (width 0.4) (layer B.Cu) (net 37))
 (segment (start 140.96 90.64) (end 147.79 90.64) (width 0.4) (layer B.Cu) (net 37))
 (segment (start 139.16 88.84) (end 140.96 90.64) (width 0.4) (layer B.Cu) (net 37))
 (segment (start 124 88.84) (end 125.41 90.25) (width 0.4) (layer B.Cu) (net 36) (status 400000))
 (segment (start 176.33 74.75) (end 177.62 73.46) (width 0.4) (layer B.Cu) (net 36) (status 800000))
 (segment (start 159.6 74.75) (end 176.33 74.75) (width 0.4) (layer B.Cu) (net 36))
 (segment (start 157.030006 77.319994) (end 159.6 74.75) (width 0.4) (layer B.Cu) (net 36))
 (segment (start 157.030006 82.248524) (end 157.030006 77.319994) (width 0.4) (layer B.Cu) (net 36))
 (segment (start 148.038528 91.240002) (end 157.030006 82.248524) (width 0.4) (layer B.Cu) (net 36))
 (segment (start 140.711472 91.240002) (end 148.038528 91.240002) (width 0.4) (layer B.Cu) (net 36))
 (segment (start 139.72147 90.25) (end 140.711472 91.240002) (width 0.4) (layer B.Cu) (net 36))
 (segment (start 125.41 90.25) (end 139.72147 90.25) (width 0.4) (layer B.Cu) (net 36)))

